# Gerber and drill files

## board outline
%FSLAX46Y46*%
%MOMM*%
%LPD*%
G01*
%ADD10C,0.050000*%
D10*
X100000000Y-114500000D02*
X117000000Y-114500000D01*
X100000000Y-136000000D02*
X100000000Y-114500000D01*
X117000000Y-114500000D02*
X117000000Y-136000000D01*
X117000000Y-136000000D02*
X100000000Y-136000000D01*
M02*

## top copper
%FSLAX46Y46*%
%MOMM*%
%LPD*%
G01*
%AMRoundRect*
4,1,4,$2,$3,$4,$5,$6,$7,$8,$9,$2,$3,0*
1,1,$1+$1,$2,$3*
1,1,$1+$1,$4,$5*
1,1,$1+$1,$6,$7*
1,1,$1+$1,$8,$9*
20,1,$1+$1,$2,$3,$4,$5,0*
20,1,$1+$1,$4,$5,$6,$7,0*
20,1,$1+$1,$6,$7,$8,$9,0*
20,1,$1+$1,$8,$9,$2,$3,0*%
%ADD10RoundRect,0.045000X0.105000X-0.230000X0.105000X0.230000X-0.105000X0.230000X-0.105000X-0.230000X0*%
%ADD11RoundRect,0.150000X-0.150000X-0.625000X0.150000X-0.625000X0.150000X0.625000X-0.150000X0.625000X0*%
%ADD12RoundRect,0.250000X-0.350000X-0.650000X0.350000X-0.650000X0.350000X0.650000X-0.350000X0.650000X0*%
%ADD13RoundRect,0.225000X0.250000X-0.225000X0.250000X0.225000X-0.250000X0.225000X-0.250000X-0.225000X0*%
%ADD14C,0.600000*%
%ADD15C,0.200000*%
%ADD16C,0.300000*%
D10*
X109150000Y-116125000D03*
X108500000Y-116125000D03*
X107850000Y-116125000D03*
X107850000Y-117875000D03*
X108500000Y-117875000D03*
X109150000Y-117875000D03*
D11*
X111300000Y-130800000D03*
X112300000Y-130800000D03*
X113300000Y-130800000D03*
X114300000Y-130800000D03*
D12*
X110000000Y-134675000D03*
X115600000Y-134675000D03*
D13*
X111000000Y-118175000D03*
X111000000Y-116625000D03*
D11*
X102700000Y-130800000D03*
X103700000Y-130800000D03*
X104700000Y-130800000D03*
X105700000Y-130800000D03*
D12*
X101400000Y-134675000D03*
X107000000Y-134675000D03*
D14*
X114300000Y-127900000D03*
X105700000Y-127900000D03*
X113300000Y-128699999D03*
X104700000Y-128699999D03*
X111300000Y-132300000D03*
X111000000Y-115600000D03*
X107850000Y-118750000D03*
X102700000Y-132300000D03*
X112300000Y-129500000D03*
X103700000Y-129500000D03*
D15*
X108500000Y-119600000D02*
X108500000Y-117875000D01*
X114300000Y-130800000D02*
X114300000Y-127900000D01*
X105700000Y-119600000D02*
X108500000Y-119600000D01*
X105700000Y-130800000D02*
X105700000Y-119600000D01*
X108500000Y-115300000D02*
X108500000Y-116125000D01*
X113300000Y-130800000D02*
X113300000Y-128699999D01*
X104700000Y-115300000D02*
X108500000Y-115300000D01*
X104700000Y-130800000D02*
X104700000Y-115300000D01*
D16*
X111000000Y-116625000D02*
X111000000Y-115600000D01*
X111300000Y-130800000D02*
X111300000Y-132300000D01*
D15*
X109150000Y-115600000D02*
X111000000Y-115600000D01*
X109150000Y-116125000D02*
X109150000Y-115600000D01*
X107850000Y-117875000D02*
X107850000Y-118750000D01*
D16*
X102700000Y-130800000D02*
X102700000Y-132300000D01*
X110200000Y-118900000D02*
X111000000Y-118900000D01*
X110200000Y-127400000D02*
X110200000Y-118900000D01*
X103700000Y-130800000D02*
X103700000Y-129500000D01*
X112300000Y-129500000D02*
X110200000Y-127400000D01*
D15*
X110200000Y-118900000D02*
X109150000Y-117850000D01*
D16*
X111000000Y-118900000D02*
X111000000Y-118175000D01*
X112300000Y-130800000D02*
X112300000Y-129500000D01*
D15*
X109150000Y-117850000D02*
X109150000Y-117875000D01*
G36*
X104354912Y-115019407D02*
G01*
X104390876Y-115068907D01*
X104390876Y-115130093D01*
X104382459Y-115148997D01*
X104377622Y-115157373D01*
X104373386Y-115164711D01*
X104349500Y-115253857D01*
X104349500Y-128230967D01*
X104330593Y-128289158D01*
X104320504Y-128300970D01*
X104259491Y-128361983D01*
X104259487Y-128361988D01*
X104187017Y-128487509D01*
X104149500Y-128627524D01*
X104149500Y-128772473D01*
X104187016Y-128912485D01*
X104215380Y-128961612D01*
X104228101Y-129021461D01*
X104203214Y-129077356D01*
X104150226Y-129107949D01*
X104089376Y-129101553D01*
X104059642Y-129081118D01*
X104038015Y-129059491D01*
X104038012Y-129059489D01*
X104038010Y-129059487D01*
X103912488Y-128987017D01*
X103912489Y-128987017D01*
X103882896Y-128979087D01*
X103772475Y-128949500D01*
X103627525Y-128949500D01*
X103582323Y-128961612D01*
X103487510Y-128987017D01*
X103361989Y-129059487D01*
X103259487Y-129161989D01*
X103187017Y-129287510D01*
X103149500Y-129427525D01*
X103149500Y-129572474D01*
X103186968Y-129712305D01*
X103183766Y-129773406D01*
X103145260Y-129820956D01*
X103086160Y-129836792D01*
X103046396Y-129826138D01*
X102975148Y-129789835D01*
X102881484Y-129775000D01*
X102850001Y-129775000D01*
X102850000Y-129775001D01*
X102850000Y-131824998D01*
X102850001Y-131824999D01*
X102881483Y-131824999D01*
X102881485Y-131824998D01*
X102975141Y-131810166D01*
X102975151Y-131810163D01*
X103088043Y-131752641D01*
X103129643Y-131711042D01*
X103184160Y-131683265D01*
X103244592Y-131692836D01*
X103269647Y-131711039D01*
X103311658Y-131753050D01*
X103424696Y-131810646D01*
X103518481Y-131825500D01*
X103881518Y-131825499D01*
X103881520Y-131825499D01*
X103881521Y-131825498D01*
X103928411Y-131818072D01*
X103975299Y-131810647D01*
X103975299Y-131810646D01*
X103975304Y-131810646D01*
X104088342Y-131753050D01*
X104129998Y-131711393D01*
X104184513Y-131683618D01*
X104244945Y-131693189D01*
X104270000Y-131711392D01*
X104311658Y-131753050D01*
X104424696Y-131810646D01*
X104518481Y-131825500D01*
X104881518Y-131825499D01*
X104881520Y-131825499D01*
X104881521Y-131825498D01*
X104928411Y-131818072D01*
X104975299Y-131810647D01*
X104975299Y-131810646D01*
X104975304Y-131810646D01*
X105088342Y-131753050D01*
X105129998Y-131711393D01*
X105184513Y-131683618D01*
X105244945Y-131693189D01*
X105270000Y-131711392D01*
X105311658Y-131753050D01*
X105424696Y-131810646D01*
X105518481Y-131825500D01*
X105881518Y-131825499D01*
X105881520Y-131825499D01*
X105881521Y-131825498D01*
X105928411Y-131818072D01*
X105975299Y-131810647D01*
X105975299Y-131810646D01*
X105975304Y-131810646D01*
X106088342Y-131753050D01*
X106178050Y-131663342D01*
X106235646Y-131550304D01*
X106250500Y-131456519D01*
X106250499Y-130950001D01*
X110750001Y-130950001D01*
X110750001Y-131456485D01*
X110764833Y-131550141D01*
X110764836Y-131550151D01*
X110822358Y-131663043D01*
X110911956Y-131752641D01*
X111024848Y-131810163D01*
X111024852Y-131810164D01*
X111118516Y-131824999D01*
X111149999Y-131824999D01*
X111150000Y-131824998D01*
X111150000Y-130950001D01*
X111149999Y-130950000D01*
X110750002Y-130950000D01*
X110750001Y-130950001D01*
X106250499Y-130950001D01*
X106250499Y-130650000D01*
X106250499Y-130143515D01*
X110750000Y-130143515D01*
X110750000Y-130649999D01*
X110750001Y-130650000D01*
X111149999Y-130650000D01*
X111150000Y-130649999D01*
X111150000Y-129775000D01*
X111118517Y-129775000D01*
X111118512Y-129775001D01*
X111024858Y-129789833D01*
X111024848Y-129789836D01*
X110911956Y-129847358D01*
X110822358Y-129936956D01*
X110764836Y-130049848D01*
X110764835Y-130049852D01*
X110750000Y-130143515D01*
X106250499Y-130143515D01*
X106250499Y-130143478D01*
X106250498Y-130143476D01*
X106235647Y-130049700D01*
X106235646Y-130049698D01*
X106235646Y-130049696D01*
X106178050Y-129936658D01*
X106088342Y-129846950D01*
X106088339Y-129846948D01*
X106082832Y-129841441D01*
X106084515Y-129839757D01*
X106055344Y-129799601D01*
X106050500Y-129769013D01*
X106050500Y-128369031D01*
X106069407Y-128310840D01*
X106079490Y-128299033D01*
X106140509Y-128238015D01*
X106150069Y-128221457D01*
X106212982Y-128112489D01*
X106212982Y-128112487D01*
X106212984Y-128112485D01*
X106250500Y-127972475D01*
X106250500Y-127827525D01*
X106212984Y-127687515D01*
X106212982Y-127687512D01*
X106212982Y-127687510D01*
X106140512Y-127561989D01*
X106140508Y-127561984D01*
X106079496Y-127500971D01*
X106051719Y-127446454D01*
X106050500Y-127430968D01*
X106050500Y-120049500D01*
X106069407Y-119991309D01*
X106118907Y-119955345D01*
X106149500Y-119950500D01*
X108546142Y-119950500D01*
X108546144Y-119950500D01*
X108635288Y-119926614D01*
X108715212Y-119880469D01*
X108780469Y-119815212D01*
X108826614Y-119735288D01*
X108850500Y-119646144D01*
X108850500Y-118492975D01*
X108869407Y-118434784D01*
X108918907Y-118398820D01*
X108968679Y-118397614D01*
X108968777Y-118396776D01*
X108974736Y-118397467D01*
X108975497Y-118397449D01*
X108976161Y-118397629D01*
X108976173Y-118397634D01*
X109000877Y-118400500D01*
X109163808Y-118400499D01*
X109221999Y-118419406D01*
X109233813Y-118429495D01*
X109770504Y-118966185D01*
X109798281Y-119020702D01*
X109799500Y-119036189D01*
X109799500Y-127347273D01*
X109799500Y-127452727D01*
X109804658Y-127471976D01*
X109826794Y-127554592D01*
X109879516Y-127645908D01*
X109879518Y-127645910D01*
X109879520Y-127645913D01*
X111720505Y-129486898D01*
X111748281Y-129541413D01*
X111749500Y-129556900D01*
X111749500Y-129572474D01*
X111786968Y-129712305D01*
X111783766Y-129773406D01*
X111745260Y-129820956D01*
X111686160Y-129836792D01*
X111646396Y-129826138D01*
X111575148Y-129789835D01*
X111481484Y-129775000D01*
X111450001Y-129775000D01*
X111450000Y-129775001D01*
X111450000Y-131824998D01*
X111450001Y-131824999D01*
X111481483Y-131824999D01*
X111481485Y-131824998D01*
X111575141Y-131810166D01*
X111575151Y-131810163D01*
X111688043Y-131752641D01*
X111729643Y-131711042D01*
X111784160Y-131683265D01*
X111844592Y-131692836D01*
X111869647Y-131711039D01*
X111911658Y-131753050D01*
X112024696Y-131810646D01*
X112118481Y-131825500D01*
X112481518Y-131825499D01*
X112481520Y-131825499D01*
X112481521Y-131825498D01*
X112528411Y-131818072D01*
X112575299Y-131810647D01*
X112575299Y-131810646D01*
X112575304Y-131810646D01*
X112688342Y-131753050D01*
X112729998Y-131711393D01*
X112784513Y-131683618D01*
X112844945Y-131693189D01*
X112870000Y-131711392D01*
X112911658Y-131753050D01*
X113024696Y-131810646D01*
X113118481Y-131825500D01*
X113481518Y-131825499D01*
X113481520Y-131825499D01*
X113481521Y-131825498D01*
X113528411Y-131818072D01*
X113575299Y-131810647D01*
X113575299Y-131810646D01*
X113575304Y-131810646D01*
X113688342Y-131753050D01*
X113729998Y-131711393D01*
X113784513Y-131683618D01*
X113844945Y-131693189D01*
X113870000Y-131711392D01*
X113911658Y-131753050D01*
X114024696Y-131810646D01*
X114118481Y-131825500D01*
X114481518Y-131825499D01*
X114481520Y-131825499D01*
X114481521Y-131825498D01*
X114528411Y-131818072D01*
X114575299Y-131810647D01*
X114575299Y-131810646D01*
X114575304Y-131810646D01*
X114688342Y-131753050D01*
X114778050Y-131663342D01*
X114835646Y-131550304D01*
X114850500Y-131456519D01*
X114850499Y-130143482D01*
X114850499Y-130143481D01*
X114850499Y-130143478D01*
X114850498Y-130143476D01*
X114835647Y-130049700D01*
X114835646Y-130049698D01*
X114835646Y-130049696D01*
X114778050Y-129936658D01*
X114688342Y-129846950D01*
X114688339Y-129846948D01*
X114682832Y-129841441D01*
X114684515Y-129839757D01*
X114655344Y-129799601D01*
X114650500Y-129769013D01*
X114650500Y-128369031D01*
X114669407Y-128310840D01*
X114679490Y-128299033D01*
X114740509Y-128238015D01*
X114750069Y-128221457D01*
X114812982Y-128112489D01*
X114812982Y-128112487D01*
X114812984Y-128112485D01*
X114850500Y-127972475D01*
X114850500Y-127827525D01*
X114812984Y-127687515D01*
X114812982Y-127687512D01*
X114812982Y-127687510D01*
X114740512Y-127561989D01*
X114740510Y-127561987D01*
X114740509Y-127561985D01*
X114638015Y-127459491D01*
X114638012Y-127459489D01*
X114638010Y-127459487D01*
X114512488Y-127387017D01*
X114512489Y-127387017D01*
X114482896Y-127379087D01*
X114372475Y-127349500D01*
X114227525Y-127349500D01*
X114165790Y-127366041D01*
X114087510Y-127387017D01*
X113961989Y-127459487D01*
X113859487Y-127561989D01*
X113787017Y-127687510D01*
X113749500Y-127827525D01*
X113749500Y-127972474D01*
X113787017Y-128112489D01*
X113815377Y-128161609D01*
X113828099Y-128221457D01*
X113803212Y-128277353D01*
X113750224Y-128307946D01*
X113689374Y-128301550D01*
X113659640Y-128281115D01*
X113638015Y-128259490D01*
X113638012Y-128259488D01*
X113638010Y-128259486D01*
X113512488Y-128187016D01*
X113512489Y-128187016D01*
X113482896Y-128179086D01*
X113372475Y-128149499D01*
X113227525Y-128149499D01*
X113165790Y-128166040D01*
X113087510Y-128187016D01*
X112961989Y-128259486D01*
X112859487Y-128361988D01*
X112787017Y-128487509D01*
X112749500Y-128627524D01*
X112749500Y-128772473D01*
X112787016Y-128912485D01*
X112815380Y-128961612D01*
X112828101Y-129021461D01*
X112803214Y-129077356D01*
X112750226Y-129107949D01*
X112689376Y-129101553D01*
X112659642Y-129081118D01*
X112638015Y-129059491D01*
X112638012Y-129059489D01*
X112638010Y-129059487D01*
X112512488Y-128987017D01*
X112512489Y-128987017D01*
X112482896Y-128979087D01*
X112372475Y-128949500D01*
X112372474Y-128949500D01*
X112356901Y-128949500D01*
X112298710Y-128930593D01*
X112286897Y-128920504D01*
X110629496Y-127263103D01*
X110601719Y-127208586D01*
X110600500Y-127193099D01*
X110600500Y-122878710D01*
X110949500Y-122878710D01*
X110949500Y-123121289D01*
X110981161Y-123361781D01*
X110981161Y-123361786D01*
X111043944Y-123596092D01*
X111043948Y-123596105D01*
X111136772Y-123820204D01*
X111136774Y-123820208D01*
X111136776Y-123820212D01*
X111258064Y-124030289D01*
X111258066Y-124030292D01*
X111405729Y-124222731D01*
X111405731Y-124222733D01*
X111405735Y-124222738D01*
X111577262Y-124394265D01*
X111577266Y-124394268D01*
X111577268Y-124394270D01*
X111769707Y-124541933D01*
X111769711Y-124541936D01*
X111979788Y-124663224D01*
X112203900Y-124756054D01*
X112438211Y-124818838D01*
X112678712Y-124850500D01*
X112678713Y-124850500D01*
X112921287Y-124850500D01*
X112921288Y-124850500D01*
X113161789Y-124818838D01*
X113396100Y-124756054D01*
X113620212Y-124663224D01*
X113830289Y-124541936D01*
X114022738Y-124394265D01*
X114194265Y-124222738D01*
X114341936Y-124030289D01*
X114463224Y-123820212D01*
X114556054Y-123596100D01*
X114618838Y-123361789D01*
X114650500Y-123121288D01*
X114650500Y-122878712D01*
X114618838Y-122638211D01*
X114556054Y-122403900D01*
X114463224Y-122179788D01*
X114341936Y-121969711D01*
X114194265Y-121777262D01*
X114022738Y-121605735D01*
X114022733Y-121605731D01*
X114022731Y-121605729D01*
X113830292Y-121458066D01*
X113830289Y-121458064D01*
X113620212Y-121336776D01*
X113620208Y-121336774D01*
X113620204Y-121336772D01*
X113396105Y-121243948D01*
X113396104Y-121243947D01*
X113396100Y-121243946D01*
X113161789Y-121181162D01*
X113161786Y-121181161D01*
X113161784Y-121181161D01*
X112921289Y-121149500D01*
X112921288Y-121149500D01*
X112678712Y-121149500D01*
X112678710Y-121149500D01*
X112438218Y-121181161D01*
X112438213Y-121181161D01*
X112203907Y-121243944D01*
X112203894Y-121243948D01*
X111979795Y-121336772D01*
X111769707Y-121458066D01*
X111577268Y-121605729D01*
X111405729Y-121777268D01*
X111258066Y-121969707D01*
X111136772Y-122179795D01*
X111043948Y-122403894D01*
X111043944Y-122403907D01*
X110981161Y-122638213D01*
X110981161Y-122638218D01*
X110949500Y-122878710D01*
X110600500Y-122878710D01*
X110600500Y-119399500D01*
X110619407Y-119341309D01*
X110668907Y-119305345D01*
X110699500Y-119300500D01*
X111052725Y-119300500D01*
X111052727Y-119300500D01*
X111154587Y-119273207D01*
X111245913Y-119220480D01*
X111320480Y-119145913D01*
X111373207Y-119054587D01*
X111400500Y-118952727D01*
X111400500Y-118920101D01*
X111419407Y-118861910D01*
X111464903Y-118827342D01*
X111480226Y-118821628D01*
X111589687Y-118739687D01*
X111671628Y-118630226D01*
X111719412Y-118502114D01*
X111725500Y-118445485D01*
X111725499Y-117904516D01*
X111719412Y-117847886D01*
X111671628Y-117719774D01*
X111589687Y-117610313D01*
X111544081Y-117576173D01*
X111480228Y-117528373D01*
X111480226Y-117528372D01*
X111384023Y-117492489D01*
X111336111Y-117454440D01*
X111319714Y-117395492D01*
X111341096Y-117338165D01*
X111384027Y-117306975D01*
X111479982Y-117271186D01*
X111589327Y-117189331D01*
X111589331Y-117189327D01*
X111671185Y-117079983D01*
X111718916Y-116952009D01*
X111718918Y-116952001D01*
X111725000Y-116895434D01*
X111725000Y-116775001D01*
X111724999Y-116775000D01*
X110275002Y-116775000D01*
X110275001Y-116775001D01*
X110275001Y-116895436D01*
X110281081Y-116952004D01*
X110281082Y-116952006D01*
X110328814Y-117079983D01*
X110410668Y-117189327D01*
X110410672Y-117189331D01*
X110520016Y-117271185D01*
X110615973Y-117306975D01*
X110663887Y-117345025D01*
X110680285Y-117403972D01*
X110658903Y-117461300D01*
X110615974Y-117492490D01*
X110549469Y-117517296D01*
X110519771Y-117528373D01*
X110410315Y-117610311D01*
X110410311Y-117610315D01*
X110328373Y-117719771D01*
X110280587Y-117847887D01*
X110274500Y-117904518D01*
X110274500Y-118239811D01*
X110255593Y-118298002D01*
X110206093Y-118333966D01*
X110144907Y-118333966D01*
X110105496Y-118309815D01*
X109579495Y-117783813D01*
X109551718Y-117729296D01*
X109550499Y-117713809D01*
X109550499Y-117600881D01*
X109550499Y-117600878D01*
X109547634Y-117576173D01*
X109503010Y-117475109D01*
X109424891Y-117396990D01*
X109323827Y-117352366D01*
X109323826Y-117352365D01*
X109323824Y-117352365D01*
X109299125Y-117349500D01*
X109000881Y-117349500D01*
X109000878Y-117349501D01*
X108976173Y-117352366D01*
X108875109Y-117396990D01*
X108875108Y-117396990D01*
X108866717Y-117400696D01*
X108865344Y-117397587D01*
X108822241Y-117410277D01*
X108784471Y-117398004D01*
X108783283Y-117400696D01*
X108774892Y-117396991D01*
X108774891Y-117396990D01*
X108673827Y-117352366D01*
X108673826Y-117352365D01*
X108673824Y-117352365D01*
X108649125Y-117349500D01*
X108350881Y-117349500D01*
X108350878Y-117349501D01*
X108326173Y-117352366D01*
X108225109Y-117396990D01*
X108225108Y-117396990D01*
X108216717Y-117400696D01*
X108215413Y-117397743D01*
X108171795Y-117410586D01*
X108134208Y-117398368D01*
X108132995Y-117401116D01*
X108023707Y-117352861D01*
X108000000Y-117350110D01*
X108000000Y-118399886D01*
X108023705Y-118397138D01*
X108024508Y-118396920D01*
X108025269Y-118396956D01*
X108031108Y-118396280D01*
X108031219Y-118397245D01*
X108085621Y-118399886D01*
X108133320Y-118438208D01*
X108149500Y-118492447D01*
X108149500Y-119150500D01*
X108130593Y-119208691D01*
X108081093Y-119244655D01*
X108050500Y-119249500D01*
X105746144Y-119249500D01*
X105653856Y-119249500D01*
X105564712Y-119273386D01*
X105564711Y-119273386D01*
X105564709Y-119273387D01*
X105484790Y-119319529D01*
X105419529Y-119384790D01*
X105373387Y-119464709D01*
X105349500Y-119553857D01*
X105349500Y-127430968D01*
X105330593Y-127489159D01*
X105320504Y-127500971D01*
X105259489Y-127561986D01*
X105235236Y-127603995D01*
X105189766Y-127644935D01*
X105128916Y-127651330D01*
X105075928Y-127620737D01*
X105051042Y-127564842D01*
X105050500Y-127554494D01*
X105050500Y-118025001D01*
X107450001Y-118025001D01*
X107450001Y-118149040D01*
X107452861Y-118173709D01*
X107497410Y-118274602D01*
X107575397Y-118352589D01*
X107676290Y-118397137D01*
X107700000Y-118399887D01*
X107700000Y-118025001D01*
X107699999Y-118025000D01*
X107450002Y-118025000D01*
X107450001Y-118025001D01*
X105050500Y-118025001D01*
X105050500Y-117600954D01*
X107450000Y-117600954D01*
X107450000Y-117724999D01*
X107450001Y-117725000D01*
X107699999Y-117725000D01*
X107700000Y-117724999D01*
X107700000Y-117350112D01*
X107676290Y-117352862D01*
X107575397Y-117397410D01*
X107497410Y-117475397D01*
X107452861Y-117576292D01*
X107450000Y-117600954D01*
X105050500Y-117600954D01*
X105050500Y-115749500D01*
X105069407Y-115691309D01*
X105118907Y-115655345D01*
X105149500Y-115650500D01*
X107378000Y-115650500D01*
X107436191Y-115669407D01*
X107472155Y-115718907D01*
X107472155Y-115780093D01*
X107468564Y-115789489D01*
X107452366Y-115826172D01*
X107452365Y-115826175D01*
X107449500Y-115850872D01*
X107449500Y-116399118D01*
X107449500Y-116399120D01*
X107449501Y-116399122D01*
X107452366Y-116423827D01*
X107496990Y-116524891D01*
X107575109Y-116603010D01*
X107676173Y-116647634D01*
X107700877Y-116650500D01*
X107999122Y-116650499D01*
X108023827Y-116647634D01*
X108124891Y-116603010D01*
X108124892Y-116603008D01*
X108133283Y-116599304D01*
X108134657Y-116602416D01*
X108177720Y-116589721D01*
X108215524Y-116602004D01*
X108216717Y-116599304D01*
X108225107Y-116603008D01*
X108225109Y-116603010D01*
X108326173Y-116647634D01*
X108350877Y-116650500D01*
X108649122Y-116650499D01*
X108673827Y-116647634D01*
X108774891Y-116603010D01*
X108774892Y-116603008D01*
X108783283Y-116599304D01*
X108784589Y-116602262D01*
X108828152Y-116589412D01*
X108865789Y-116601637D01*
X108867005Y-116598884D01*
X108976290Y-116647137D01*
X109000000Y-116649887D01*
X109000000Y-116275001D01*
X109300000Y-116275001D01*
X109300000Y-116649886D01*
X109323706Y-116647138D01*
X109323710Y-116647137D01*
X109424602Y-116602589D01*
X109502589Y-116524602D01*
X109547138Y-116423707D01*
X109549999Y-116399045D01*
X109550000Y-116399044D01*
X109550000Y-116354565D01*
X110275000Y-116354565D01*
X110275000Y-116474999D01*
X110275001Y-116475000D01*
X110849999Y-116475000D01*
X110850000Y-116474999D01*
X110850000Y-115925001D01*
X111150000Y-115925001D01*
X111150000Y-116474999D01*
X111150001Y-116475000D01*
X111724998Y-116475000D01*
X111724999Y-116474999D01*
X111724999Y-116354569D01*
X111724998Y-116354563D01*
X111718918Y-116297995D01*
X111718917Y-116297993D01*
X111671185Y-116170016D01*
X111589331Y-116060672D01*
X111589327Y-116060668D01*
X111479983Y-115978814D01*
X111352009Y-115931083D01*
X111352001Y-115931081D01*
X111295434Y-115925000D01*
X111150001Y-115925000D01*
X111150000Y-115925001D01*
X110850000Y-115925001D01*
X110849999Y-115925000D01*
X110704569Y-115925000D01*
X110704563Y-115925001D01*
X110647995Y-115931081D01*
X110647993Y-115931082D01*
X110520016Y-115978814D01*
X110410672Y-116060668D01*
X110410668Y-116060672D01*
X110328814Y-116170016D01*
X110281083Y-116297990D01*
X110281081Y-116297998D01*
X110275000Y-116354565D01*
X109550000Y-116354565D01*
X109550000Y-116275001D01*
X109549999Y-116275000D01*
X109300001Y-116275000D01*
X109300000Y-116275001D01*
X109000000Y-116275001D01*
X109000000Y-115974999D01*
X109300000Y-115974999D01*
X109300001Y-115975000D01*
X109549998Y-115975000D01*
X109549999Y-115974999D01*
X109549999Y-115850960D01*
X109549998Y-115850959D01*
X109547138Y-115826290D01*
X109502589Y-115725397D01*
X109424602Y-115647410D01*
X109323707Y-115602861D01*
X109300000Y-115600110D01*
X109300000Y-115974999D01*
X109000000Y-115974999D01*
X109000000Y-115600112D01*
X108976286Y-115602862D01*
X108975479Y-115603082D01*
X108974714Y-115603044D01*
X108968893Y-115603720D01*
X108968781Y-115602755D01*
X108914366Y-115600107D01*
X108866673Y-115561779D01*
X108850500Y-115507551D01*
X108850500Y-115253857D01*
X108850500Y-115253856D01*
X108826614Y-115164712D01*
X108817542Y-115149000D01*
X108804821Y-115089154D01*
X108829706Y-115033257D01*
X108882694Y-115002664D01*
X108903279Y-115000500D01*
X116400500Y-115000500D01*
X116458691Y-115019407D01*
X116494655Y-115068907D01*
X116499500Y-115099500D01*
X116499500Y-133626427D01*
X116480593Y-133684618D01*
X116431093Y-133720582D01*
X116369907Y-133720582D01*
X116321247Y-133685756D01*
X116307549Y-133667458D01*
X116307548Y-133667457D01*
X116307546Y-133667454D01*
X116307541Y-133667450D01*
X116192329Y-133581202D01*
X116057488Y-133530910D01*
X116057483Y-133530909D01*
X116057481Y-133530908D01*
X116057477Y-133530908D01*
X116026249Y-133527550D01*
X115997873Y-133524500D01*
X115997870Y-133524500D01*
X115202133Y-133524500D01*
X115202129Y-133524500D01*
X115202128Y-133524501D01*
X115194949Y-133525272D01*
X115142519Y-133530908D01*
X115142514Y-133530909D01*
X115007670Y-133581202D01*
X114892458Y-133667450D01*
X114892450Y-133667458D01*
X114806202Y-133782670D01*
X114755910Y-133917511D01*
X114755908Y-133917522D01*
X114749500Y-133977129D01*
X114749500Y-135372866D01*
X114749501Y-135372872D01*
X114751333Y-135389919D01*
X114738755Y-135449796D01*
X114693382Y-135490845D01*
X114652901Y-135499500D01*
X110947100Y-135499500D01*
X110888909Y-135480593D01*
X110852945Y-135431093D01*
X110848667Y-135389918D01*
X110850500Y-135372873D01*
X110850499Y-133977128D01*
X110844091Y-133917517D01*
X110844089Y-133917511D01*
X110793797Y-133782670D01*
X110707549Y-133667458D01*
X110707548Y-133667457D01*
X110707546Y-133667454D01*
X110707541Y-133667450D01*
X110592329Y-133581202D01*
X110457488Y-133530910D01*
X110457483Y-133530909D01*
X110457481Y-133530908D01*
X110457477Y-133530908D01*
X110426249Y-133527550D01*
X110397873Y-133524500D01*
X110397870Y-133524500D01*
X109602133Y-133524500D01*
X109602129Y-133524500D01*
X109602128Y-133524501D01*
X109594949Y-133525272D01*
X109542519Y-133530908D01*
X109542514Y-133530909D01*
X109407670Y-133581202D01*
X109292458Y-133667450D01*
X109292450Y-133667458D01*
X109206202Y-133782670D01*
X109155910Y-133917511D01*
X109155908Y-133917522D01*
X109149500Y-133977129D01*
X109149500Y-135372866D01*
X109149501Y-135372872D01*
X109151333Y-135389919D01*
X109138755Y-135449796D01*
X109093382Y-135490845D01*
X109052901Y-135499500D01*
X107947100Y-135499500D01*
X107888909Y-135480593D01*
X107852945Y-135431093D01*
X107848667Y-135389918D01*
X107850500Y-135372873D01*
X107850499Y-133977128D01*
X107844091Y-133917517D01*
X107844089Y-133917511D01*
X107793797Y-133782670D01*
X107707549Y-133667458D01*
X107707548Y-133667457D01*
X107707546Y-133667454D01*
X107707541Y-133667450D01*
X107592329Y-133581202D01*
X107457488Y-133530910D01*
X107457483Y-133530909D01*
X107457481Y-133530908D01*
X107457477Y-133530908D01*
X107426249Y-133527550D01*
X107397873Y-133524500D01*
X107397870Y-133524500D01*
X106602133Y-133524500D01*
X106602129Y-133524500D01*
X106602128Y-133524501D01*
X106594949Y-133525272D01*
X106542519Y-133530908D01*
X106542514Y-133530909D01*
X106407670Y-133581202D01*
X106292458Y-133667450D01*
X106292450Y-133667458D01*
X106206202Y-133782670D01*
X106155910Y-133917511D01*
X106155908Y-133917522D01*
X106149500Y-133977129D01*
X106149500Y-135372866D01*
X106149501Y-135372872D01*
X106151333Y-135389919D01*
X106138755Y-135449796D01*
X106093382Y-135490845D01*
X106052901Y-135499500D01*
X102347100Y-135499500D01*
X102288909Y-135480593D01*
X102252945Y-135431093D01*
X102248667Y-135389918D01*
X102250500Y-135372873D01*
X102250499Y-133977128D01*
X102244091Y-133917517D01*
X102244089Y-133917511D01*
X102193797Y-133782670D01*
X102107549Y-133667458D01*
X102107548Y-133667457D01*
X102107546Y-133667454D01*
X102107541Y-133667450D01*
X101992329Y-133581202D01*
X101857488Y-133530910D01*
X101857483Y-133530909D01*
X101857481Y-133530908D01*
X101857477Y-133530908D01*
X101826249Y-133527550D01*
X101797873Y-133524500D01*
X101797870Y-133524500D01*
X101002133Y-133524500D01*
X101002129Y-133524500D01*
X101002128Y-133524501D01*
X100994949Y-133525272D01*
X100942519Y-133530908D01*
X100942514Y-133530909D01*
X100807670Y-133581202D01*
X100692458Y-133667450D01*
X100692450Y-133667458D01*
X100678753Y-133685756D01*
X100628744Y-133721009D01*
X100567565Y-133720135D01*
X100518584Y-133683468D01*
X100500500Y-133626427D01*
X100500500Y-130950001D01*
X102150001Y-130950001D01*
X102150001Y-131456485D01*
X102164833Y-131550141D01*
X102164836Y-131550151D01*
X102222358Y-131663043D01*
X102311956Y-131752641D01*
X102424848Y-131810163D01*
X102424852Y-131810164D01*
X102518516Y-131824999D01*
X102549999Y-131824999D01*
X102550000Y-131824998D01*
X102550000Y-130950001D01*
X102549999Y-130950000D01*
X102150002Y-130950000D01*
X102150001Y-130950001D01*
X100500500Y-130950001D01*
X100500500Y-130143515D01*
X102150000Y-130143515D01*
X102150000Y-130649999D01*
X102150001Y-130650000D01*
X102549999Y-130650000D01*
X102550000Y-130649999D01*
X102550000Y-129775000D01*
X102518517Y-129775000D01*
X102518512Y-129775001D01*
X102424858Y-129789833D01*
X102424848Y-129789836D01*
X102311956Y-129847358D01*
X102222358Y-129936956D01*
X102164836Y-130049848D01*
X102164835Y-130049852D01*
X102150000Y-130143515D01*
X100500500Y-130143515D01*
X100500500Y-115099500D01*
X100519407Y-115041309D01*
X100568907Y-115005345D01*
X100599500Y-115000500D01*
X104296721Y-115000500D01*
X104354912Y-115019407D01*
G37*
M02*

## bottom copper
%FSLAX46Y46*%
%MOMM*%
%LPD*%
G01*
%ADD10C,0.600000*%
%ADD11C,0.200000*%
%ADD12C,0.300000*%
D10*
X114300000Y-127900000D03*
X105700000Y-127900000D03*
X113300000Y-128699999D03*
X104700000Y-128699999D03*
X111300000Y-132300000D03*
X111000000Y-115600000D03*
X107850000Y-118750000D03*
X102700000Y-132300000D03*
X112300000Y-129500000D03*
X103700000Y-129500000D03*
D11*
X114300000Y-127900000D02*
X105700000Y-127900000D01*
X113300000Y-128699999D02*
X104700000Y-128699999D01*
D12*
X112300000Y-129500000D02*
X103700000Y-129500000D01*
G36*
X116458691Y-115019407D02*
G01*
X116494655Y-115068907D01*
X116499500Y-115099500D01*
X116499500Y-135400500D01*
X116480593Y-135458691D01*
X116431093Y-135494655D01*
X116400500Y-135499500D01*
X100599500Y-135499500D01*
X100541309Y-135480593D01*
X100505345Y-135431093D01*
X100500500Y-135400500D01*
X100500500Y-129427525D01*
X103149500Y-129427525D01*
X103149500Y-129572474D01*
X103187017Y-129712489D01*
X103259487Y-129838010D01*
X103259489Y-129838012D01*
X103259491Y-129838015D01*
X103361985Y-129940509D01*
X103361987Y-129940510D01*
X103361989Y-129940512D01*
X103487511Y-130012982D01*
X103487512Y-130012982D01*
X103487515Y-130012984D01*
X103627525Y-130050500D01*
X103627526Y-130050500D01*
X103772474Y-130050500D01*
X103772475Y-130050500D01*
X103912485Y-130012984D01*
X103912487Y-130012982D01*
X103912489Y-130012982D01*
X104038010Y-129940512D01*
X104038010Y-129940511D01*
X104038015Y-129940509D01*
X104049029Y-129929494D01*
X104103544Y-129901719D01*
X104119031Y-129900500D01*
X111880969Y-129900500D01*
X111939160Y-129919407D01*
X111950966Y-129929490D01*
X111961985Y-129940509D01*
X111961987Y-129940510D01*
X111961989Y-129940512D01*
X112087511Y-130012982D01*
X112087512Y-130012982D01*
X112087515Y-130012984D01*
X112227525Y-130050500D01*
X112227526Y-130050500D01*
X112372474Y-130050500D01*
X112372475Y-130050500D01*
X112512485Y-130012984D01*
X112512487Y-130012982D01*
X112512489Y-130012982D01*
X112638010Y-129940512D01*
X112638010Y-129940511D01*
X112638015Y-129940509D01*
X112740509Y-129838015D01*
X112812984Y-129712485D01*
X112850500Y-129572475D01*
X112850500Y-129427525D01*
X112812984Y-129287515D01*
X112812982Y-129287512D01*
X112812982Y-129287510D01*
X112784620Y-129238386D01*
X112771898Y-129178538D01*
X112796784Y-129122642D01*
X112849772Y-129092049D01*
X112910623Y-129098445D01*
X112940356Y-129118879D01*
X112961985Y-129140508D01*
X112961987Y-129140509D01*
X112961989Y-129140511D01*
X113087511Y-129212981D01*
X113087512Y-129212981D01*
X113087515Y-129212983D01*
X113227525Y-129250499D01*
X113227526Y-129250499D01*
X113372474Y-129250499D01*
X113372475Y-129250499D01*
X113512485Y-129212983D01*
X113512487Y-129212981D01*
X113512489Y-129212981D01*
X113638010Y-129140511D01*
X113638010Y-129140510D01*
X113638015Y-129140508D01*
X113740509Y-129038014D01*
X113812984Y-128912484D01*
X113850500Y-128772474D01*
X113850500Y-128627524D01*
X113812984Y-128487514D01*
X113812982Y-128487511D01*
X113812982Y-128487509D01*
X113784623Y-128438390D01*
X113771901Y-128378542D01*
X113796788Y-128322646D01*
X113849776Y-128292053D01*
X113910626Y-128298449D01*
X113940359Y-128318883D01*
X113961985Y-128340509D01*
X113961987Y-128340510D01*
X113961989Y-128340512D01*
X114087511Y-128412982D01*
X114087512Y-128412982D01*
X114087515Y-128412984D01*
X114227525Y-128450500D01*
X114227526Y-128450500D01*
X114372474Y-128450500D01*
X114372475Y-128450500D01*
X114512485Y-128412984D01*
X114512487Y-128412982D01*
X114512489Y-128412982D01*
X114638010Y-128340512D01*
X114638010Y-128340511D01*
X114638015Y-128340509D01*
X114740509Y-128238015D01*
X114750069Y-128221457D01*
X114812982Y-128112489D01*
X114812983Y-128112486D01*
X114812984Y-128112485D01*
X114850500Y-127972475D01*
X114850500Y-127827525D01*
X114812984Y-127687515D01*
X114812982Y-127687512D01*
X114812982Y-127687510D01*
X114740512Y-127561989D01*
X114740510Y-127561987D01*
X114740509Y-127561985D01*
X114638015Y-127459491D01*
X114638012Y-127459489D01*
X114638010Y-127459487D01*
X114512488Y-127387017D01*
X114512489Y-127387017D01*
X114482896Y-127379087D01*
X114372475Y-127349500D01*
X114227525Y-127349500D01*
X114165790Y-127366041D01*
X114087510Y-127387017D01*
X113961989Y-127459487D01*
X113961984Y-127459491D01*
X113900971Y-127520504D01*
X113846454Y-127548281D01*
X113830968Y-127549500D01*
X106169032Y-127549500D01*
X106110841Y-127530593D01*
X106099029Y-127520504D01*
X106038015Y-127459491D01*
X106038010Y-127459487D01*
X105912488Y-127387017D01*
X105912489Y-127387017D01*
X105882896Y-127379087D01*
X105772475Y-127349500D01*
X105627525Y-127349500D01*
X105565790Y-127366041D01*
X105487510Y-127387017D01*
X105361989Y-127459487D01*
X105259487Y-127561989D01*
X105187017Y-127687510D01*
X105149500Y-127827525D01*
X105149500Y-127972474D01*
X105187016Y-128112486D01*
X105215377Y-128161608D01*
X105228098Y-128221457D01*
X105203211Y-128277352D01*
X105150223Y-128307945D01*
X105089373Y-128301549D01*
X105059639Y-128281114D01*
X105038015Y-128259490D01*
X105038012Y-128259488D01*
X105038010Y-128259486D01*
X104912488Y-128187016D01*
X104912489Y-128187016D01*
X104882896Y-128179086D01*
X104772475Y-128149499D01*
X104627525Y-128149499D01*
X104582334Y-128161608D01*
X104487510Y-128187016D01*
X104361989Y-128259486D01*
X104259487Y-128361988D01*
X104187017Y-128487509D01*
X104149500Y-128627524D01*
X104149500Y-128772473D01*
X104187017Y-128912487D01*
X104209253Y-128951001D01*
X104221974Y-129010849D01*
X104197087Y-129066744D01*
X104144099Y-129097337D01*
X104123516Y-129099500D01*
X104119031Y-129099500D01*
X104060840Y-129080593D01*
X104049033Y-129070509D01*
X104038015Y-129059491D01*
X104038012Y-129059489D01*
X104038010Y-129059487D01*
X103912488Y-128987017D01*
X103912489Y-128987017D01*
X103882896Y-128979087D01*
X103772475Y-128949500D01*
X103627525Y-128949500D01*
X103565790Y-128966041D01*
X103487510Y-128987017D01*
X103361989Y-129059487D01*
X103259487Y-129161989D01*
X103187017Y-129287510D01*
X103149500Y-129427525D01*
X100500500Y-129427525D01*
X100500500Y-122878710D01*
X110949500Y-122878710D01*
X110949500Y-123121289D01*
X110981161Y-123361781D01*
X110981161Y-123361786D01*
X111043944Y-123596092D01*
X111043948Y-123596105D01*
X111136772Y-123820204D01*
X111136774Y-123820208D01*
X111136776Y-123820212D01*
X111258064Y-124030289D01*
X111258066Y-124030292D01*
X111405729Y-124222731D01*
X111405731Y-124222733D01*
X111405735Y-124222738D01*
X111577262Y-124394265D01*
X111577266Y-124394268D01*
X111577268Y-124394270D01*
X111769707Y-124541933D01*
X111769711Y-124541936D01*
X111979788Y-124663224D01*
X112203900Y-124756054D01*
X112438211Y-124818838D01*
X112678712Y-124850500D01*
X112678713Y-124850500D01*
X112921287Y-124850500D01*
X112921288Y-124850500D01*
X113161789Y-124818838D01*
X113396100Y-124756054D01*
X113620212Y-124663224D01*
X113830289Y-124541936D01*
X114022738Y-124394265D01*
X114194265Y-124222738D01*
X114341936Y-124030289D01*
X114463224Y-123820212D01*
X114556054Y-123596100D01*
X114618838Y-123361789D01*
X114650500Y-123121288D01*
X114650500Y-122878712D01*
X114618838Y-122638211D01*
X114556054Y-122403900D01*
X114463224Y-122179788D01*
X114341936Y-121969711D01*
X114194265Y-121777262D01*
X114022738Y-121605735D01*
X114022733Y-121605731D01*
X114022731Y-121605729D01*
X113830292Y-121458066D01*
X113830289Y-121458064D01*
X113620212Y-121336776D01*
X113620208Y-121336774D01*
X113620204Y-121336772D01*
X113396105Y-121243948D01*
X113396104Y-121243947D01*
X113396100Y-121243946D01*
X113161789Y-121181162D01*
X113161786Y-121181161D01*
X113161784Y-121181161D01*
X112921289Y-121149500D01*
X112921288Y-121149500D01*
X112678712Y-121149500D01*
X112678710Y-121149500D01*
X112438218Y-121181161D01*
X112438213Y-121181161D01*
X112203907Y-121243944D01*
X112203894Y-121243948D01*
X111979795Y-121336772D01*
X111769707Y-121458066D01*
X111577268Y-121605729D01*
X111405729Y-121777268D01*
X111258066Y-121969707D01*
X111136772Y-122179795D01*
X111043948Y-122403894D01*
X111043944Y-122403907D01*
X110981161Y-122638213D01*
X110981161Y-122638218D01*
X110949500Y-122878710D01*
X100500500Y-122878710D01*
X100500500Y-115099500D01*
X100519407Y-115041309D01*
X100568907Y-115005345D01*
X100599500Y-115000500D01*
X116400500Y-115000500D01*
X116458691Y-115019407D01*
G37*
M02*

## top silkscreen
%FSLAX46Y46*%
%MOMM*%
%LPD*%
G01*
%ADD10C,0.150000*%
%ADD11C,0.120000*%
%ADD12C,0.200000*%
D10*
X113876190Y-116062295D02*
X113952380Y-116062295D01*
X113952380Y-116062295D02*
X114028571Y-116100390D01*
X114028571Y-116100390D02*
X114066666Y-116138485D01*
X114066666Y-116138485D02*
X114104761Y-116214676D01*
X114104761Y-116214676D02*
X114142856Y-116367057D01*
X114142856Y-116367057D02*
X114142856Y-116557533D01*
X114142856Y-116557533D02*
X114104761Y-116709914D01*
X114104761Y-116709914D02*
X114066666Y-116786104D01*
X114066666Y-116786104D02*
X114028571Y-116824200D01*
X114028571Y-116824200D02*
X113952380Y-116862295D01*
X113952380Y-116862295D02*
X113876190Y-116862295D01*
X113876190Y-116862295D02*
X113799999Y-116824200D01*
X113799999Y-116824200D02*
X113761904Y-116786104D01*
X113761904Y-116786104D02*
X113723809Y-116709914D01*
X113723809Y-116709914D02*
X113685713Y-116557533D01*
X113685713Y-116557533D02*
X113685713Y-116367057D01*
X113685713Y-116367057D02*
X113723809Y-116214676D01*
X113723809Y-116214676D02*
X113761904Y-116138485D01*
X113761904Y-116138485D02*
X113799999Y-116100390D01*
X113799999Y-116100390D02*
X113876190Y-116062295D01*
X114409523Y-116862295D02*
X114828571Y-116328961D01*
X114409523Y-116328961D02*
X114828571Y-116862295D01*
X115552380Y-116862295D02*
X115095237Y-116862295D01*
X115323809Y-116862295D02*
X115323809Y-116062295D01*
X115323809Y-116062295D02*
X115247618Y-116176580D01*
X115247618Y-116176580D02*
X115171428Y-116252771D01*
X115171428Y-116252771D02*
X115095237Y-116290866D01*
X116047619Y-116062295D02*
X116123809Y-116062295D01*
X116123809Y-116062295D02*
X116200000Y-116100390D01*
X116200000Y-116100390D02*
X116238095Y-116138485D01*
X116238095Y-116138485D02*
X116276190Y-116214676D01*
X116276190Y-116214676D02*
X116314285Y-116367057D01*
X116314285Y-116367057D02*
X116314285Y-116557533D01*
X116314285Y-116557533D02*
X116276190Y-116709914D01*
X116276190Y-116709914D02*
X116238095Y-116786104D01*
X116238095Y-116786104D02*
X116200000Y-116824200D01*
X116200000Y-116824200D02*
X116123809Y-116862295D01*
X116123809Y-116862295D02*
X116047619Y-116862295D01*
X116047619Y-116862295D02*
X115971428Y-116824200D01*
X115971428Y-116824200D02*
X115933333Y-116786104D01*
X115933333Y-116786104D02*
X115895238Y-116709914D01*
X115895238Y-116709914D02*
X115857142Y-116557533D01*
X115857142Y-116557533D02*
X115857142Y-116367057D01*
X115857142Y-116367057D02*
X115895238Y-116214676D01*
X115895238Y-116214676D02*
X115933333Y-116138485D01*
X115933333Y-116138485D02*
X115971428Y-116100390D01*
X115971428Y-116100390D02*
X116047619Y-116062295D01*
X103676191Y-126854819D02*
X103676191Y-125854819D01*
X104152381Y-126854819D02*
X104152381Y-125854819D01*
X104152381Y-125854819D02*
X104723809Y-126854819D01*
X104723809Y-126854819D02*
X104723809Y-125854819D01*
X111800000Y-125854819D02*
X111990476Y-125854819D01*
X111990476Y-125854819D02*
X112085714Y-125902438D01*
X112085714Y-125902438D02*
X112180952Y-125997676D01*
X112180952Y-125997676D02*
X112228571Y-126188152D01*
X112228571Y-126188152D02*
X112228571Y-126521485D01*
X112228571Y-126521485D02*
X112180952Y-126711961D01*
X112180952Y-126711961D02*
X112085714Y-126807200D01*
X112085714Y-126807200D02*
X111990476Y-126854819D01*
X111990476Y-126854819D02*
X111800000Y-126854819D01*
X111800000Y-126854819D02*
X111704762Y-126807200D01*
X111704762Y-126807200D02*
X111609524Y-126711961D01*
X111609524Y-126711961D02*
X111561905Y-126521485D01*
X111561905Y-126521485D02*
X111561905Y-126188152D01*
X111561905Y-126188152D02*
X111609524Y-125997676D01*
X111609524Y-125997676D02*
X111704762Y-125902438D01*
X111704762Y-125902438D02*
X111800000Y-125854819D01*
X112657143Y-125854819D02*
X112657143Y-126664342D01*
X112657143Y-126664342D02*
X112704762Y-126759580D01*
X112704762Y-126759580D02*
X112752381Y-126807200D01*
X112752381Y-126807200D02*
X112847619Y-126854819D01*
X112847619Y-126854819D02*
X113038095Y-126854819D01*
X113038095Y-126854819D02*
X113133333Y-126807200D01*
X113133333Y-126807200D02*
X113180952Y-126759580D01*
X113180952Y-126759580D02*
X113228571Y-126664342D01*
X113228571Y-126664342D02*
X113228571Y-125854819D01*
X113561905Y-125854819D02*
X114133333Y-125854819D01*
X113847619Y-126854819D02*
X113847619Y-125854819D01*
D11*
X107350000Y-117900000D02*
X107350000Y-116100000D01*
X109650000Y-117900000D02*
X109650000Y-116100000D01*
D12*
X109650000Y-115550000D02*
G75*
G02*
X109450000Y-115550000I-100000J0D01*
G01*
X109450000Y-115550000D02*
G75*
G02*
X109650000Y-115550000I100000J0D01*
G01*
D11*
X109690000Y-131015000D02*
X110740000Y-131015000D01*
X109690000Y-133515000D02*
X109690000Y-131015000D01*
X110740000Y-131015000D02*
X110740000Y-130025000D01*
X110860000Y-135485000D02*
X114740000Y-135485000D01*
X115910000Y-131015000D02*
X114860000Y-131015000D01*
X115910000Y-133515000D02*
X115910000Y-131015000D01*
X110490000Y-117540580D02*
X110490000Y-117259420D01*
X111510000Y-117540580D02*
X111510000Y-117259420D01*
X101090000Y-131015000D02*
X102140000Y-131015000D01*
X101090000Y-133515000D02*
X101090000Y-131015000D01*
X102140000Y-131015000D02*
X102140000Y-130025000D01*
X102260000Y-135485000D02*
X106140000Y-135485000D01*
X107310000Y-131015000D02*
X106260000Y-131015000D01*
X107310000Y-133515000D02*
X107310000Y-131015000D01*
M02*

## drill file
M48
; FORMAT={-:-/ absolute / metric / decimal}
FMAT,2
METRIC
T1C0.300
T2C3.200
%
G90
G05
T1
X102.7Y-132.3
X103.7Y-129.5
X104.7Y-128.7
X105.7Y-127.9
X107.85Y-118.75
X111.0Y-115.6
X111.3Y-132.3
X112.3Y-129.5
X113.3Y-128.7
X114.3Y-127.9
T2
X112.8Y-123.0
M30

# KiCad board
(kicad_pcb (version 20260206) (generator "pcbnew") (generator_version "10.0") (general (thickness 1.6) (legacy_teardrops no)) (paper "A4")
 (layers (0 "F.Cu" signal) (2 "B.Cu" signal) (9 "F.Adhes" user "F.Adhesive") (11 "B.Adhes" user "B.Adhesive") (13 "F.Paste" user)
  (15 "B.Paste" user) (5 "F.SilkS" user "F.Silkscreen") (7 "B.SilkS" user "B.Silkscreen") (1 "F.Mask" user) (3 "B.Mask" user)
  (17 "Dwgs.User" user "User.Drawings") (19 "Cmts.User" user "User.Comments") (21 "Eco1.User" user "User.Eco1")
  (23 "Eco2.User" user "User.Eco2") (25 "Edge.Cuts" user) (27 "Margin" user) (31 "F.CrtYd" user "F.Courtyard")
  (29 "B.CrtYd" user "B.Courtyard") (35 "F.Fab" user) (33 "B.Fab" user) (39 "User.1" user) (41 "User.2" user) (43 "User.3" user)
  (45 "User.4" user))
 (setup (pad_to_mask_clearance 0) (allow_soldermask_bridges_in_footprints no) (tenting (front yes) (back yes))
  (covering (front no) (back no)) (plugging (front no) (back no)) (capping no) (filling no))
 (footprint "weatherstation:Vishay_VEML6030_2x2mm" (layer "F.Cu") (at 108.5 117 90)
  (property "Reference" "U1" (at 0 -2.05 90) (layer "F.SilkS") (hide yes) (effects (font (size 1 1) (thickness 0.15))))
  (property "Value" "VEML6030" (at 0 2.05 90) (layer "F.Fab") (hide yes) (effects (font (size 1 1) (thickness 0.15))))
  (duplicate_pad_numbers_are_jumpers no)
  (fp_line (start -0.9 -1.15) (end 0.9 -1.15) (stroke (width 0.12) (type default)) (layer "F.SilkS"))
  (fp_line (start -0.9 1.15) (end 0.9 1.15) (stroke (width 0.12) (type default)) (layer "F.SilkS"))
  (fp_circle (center 1.45 1.05) (end 1.55 1.05) (stroke (width 0.2) (type default)) (fill yes) (layer "F.SilkS"))
  (pad "1" smd roundrect (at 0.875 0.65 90) (size 0.55 0.3) (layers "F.Cu" "F.Mask" "F.Paste") (roundrect_rratio 0.15) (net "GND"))
  (pad "2" smd roundrect (at 0.875 0 90) (size 0.55 0.3) (layers "F.Cu" "F.Mask" "F.Paste") (roundrect_rratio 0.15) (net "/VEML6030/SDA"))
  (pad "3" smd roundrect (at 0.875 -0.65 90) (size 0.55 0.3) (layers "F.Cu" "F.Mask" "F.Paste") (roundrect_rratio 0.15)
   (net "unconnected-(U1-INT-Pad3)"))
  (pad "4" smd roundrect (at -0.875 -0.65 90) (size 0.55 0.3) (layers "F.Cu" "F.Mask" "F.Paste") (roundrect_rratio 0.15) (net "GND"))
  (pad "5" smd roundrect (at -0.875 0 90) (size 0.55 0.3) (layers "F.Cu" "F.Mask" "F.Paste") (roundrect_rratio 0.15) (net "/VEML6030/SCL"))
  (pad "6" smd roundrect (at -0.875 0.65 90) (size 0.55 0.3) (layers "F.Cu" "F.Mask" "F.Paste") (roundrect_rratio 0.15) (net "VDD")))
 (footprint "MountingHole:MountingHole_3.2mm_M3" (layer "F.Cu") (at 112.8 123)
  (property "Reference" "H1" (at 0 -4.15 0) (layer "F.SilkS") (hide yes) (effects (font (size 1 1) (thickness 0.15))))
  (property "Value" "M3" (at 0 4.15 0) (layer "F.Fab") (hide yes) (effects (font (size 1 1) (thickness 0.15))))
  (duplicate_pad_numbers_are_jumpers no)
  (pad "" np_thru_hole circle (at 0 0) (size 3.2 3.2) (drill 3.2) (layers "*.Cu" "*.Mask")))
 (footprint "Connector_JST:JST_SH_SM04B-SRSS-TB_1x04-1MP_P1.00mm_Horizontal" (layer "F.Cu") (at 112.8 132.8)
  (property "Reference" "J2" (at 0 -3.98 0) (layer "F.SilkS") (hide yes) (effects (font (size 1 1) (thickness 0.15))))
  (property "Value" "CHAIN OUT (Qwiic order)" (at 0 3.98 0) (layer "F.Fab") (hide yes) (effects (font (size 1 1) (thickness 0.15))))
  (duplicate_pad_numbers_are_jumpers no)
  (fp_line (start -3.11 -1.785) (end -2.06 -1.785) (stroke (width 0.12) (type solid)) (layer "F.SilkS"))
  (fp_line (start -3.11 0.715) (end -3.11 -1.785) (stroke (width 0.12) (type solid)) (layer "F.SilkS"))
  (fp_line (start -2.06 -1.785) (end -2.06 -2.775) (stroke (width 0.12) (type solid)) (layer "F.SilkS"))
  (fp_line (start -1.94 2.685) (end 1.94 2.685) (stroke (width 0.12) (type solid)) (layer "F.SilkS"))
  (fp_line (start 3.11 -1.785) (end 2.06 -1.785) (stroke (width 0.12) (type solid)) (layer "F.SilkS"))
  (fp_line (start 3.11 0.715) (end 3.11 -1.785) (stroke (width 0.12) (type solid)) (layer "F.SilkS"))
  (pad "1" smd roundrect (at -1.5 -2) (size 0.6 1.55) (layers "F.Cu" "F.Mask" "F.Paste") (roundrect_rratio 0.25) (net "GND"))
  (pad "2" smd roundrect (at -0.5 -2) (size 0.6 1.55) (layers "F.Cu" "F.Mask" "F.Paste") (roundrect_rratio 0.25) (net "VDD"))
  (pad "3" smd roundrect (at 0.5 -2) (size 0.6 1.55) (layers "F.Cu" "F.Mask" "F.Paste") (roundrect_rratio 0.25) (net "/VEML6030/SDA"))
  (pad "4" smd roundrect (at 1.5 -2) (size 0.6 1.55) (layers "F.Cu" "F.Mask" "F.Paste") (roundrect_rratio 0.25) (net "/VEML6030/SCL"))
  (pad "MP" smd roundrect (at -2.8 1.875) (size 1.2 1.8) (layers "F.Cu" "F.Mask" "F.Paste") (roundrect_rratio 0.208333))
  (pad "MP" smd roundrect (at 2.8 1.875) (size 1.2 1.8) (layers "F.Cu" "F.Mask" "F.Paste") (roundrect_rratio 0.208333)))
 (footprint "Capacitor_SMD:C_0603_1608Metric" (layer "F.Cu") (at 111 117.4 90)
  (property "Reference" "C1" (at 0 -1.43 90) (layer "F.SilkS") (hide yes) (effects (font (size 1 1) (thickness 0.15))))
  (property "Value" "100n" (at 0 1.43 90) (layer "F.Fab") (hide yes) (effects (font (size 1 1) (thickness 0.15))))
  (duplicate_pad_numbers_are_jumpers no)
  (fp_line (start -0.14058 -0.51) (end 0.14058 -0.51) (stroke (width 0.12) (type solid)) (layer "F.SilkS"))
  (fp_line (start -0.14058 0.51) (end 0.14058 0.51) (stroke (width 0.12) (type solid)) (layer "F.SilkS"))
  (pad "1" smd roundrect (at -0.775 0 90) (size 0.9 0.95) (layers "F.Cu" "F.Mask" "F.Paste") (roundrect_rratio 0.25) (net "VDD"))
  (pad "2" smd roundrect (at 0.775 0 90) (size 0.9 0.95) (layers "F.Cu" "F.Mask" "F.Paste") (roundrect_rratio 0.25) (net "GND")))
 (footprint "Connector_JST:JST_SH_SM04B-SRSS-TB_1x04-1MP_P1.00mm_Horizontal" (layer "F.Cu") (at 104.2 132.8)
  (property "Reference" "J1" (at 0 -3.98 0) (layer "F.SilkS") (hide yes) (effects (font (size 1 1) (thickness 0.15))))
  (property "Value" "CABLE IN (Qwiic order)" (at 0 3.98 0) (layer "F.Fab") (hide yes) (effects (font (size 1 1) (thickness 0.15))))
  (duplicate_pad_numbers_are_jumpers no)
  (fp_line (start -3.11 -1.785) (end -2.06 -1.785) (stroke (width 0.12) (type solid)) (layer "F.SilkS"))
  (fp_line (start -3.11 0.715) (end -3.11 -1.785) (stroke (width 0.12) (type solid)) (layer "F.SilkS"))
  (fp_line (start -2.06 -1.785) (end -2.06 -2.775) (stroke (width 0.12) (type solid)) (layer "F.SilkS"))
  (fp_line (start -1.94 2.685) (end 1.94 2.685) (stroke (width 0.12) (type solid)) (layer "F.SilkS"))
  (fp_line (start 3.11 -1.785) (end 2.06 -1.785) (stroke (width 0.12) (type solid)) (layer "F.SilkS"))
  (fp_line (start 3.11 0.715) (end 3.11 -1.785) (stroke (width 0.12) (type solid)) (layer "F.SilkS"))
  (pad "1" smd roundrect (at -1.5 -2) (size 0.6 1.55) (layers "F.Cu" "F.Mask" "F.Paste") (roundrect_rratio 0.25) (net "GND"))
  (pad "2" smd roundrect (at -0.5 -2) (size 0.6 1.55) (layers "F.Cu" "F.Mask" "F.Paste") (roundrect_rratio 0.25) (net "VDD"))
  (pad "3" smd roundrect (at 0.5 -2) (size 0.6 1.55) (layers "F.Cu" "F.Mask" "F.Paste") (roundrect_rratio 0.25) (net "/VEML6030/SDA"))
  (pad "4" smd roundrect (at 1.5 -2) (size 0.6 1.55) (layers "F.Cu" "F.Mask" "F.Paste") (roundrect_rratio 0.25) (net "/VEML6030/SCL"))
  (pad "MP" smd roundrect (at -2.8 1.875) (size 1.2 1.8) (layers "F.Cu" "F.Mask" "F.Paste") (roundrect_rratio 0.208333))
  (pad "MP" smd roundrect (at 2.8 1.875) (size 1.2 1.8) (layers "F.Cu" "F.Mask" "F.Paste") (roundrect_rratio 0.208333)))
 (gr_line (start 100 114.5) (end 117 114.5) (stroke (width 0.05) (type default)) (layer "Edge.Cuts"))
 (gr_line (start 100 136) (end 100 114.5) (stroke (width 0.05) (type default)) (layer "Edge.Cuts"))
 (gr_line (start 117 114.5) (end 117 136) (stroke (width 0.05) (type default)) (layer "Edge.Cuts"))
 (gr_line (start 117 136) (end 100 136) (stroke (width 0.05) (type default)) (layer "Edge.Cuts"))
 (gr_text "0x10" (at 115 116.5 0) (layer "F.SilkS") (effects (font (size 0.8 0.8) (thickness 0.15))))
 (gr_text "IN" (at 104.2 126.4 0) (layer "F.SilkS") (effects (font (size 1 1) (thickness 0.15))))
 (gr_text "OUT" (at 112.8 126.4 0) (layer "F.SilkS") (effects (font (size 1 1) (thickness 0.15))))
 (segment (start 108.5 119.6) (end 108.5 117.875) (width 0.2) (layer "F.Cu") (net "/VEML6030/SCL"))
 (segment (start 114.3 130.8) (end 114.3 127.9) (width 0.2) (layer "F.Cu") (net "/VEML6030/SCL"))
 (segment (start 105.7 119.6) (end 108.5 119.6) (width 0.2) (layer "F.Cu") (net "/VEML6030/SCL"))
 (segment (start 105.7 130.8) (end 105.7 119.6) (width 0.2) (layer "F.Cu") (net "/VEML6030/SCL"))
 (via (at 114.3 127.9) (size 0.6) (drill 0.3) (layers "F.Cu" "B.Cu") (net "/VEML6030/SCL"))
 (via (at 105.7 127.9) (size 0.6) (drill 0.3) (layers "F.Cu" "B.Cu") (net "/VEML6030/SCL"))
 (segment (start 114.3 127.9) (end 105.7 127.9) (width 0.2) (layer "B.Cu") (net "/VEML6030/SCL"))
 (segment (start 108.5 115.3) (end 108.5 116.125) (width 0.2) (layer "F.Cu") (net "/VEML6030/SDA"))
 (segment (start 113.3 130.8) (end 113.3 128.699999) (width 0.2) (layer "F.Cu") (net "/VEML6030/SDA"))
 (segment (start 104.7 115.3) (end 108.5 115.3) (width 0.2) (layer "F.Cu") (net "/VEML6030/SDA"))
 (segment (start 104.7 130.8) (end 104.7 115.3) (width 0.2) (layer "F.Cu") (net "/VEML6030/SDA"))
 (via (at 113.3 128.699999) (size 0.6) (drill 0.3) (layers "F.Cu" "B.Cu") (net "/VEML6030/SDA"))
 (via (at 104.7 128.699999) (size 0.6) (drill 0.3) (layers "F.Cu" "B.Cu") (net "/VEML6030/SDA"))
 (segment (start 113.3 128.699999) (end 104.7 128.699999) (width 0.2) (layer "B.Cu") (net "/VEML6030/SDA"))
 (segment (start 111 116.625) (end 111 115.6) (width 0.3) (layer "F.Cu") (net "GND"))
 (segment (start 111.3 130.8) (end 111.3 132.3) (width 0.3) (layer "F.Cu") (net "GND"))
 (segment (start 109.15 115.6) (end 111 115.6) (width 0.2) (layer "F.Cu") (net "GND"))
 (segment (start 109.15 116.125) (end 109.15 115.6) (width 0.2) (layer "F.Cu") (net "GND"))
 (segment (start 107.85 117.875) (end 107.85 118.75) (width 0.2) (layer "F.Cu") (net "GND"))
 (segment (start 102.7 130.8) (end 102.7 132.3) (width 0.3) (layer "F.Cu") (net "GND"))
 (via (at 111.3 132.3) (size 0.6) (drill 0.3) (layers "F.Cu" "B.Cu") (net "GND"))
 (via (at 111 115.6) (size 0.6) (drill 0.3) (layers "F.Cu" "B.Cu") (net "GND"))
 (via (at 107.85 118.75) (size 0.6) (drill 0.3) (layers "F.Cu" "B.Cu") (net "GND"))
 (via (at 102.7 132.3) (size 0.6) (drill 0.3) (layers "F.Cu" "B.Cu") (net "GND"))
 (segment (start 110.2 118.9) (end 111 118.9) (width 0.3) (layer "F.Cu") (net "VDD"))
 (segment (start 110.2 127.4) (end 110.2 118.9) (width 0.3) (layer "F.Cu") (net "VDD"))
 (segment (start 103.7 130.8) (end 103.7 129.5) (width 0.3) (layer "F.Cu") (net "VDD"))
 (segment (start 112.3 129.5) (end 110.2 127.4) (width 0.3) (layer "F.Cu") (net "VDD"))
 (segment (start 110.2 118.9) (end 109.15 117.85) (width 0.2) (layer "F.Cu") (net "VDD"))
 (segment (start 111 118.9) (end 111 118.175) (width 0.3) (layer "F.Cu") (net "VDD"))
 (segment (start 112.3 130.8) (end 112.3 129.5) (width 0.3) (layer "F.Cu") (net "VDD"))
 (segment (start 109.15 117.85) (end 109.15 117.875) (width 0.2) (layer "F.Cu") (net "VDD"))
 (via (at 112.3 129.5) (size 0.6) (drill 0.3) (layers "F.Cu" "B.Cu") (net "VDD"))
 (via (at 103.7 129.5) (size 0.6) (drill 0.3) (layers "F.Cu" "B.Cu") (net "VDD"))
 (segment (start 112.3 129.5) (end 103.7 129.5) (width 0.3) (layer "B.Cu") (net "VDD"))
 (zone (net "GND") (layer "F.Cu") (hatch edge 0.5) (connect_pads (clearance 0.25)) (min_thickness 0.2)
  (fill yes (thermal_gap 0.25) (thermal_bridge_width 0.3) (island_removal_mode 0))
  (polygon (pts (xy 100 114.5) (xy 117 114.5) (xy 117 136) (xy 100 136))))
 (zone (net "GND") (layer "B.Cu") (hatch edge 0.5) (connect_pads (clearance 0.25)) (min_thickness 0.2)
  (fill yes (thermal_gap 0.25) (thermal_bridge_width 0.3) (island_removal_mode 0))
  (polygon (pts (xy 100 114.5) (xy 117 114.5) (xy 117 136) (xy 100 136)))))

